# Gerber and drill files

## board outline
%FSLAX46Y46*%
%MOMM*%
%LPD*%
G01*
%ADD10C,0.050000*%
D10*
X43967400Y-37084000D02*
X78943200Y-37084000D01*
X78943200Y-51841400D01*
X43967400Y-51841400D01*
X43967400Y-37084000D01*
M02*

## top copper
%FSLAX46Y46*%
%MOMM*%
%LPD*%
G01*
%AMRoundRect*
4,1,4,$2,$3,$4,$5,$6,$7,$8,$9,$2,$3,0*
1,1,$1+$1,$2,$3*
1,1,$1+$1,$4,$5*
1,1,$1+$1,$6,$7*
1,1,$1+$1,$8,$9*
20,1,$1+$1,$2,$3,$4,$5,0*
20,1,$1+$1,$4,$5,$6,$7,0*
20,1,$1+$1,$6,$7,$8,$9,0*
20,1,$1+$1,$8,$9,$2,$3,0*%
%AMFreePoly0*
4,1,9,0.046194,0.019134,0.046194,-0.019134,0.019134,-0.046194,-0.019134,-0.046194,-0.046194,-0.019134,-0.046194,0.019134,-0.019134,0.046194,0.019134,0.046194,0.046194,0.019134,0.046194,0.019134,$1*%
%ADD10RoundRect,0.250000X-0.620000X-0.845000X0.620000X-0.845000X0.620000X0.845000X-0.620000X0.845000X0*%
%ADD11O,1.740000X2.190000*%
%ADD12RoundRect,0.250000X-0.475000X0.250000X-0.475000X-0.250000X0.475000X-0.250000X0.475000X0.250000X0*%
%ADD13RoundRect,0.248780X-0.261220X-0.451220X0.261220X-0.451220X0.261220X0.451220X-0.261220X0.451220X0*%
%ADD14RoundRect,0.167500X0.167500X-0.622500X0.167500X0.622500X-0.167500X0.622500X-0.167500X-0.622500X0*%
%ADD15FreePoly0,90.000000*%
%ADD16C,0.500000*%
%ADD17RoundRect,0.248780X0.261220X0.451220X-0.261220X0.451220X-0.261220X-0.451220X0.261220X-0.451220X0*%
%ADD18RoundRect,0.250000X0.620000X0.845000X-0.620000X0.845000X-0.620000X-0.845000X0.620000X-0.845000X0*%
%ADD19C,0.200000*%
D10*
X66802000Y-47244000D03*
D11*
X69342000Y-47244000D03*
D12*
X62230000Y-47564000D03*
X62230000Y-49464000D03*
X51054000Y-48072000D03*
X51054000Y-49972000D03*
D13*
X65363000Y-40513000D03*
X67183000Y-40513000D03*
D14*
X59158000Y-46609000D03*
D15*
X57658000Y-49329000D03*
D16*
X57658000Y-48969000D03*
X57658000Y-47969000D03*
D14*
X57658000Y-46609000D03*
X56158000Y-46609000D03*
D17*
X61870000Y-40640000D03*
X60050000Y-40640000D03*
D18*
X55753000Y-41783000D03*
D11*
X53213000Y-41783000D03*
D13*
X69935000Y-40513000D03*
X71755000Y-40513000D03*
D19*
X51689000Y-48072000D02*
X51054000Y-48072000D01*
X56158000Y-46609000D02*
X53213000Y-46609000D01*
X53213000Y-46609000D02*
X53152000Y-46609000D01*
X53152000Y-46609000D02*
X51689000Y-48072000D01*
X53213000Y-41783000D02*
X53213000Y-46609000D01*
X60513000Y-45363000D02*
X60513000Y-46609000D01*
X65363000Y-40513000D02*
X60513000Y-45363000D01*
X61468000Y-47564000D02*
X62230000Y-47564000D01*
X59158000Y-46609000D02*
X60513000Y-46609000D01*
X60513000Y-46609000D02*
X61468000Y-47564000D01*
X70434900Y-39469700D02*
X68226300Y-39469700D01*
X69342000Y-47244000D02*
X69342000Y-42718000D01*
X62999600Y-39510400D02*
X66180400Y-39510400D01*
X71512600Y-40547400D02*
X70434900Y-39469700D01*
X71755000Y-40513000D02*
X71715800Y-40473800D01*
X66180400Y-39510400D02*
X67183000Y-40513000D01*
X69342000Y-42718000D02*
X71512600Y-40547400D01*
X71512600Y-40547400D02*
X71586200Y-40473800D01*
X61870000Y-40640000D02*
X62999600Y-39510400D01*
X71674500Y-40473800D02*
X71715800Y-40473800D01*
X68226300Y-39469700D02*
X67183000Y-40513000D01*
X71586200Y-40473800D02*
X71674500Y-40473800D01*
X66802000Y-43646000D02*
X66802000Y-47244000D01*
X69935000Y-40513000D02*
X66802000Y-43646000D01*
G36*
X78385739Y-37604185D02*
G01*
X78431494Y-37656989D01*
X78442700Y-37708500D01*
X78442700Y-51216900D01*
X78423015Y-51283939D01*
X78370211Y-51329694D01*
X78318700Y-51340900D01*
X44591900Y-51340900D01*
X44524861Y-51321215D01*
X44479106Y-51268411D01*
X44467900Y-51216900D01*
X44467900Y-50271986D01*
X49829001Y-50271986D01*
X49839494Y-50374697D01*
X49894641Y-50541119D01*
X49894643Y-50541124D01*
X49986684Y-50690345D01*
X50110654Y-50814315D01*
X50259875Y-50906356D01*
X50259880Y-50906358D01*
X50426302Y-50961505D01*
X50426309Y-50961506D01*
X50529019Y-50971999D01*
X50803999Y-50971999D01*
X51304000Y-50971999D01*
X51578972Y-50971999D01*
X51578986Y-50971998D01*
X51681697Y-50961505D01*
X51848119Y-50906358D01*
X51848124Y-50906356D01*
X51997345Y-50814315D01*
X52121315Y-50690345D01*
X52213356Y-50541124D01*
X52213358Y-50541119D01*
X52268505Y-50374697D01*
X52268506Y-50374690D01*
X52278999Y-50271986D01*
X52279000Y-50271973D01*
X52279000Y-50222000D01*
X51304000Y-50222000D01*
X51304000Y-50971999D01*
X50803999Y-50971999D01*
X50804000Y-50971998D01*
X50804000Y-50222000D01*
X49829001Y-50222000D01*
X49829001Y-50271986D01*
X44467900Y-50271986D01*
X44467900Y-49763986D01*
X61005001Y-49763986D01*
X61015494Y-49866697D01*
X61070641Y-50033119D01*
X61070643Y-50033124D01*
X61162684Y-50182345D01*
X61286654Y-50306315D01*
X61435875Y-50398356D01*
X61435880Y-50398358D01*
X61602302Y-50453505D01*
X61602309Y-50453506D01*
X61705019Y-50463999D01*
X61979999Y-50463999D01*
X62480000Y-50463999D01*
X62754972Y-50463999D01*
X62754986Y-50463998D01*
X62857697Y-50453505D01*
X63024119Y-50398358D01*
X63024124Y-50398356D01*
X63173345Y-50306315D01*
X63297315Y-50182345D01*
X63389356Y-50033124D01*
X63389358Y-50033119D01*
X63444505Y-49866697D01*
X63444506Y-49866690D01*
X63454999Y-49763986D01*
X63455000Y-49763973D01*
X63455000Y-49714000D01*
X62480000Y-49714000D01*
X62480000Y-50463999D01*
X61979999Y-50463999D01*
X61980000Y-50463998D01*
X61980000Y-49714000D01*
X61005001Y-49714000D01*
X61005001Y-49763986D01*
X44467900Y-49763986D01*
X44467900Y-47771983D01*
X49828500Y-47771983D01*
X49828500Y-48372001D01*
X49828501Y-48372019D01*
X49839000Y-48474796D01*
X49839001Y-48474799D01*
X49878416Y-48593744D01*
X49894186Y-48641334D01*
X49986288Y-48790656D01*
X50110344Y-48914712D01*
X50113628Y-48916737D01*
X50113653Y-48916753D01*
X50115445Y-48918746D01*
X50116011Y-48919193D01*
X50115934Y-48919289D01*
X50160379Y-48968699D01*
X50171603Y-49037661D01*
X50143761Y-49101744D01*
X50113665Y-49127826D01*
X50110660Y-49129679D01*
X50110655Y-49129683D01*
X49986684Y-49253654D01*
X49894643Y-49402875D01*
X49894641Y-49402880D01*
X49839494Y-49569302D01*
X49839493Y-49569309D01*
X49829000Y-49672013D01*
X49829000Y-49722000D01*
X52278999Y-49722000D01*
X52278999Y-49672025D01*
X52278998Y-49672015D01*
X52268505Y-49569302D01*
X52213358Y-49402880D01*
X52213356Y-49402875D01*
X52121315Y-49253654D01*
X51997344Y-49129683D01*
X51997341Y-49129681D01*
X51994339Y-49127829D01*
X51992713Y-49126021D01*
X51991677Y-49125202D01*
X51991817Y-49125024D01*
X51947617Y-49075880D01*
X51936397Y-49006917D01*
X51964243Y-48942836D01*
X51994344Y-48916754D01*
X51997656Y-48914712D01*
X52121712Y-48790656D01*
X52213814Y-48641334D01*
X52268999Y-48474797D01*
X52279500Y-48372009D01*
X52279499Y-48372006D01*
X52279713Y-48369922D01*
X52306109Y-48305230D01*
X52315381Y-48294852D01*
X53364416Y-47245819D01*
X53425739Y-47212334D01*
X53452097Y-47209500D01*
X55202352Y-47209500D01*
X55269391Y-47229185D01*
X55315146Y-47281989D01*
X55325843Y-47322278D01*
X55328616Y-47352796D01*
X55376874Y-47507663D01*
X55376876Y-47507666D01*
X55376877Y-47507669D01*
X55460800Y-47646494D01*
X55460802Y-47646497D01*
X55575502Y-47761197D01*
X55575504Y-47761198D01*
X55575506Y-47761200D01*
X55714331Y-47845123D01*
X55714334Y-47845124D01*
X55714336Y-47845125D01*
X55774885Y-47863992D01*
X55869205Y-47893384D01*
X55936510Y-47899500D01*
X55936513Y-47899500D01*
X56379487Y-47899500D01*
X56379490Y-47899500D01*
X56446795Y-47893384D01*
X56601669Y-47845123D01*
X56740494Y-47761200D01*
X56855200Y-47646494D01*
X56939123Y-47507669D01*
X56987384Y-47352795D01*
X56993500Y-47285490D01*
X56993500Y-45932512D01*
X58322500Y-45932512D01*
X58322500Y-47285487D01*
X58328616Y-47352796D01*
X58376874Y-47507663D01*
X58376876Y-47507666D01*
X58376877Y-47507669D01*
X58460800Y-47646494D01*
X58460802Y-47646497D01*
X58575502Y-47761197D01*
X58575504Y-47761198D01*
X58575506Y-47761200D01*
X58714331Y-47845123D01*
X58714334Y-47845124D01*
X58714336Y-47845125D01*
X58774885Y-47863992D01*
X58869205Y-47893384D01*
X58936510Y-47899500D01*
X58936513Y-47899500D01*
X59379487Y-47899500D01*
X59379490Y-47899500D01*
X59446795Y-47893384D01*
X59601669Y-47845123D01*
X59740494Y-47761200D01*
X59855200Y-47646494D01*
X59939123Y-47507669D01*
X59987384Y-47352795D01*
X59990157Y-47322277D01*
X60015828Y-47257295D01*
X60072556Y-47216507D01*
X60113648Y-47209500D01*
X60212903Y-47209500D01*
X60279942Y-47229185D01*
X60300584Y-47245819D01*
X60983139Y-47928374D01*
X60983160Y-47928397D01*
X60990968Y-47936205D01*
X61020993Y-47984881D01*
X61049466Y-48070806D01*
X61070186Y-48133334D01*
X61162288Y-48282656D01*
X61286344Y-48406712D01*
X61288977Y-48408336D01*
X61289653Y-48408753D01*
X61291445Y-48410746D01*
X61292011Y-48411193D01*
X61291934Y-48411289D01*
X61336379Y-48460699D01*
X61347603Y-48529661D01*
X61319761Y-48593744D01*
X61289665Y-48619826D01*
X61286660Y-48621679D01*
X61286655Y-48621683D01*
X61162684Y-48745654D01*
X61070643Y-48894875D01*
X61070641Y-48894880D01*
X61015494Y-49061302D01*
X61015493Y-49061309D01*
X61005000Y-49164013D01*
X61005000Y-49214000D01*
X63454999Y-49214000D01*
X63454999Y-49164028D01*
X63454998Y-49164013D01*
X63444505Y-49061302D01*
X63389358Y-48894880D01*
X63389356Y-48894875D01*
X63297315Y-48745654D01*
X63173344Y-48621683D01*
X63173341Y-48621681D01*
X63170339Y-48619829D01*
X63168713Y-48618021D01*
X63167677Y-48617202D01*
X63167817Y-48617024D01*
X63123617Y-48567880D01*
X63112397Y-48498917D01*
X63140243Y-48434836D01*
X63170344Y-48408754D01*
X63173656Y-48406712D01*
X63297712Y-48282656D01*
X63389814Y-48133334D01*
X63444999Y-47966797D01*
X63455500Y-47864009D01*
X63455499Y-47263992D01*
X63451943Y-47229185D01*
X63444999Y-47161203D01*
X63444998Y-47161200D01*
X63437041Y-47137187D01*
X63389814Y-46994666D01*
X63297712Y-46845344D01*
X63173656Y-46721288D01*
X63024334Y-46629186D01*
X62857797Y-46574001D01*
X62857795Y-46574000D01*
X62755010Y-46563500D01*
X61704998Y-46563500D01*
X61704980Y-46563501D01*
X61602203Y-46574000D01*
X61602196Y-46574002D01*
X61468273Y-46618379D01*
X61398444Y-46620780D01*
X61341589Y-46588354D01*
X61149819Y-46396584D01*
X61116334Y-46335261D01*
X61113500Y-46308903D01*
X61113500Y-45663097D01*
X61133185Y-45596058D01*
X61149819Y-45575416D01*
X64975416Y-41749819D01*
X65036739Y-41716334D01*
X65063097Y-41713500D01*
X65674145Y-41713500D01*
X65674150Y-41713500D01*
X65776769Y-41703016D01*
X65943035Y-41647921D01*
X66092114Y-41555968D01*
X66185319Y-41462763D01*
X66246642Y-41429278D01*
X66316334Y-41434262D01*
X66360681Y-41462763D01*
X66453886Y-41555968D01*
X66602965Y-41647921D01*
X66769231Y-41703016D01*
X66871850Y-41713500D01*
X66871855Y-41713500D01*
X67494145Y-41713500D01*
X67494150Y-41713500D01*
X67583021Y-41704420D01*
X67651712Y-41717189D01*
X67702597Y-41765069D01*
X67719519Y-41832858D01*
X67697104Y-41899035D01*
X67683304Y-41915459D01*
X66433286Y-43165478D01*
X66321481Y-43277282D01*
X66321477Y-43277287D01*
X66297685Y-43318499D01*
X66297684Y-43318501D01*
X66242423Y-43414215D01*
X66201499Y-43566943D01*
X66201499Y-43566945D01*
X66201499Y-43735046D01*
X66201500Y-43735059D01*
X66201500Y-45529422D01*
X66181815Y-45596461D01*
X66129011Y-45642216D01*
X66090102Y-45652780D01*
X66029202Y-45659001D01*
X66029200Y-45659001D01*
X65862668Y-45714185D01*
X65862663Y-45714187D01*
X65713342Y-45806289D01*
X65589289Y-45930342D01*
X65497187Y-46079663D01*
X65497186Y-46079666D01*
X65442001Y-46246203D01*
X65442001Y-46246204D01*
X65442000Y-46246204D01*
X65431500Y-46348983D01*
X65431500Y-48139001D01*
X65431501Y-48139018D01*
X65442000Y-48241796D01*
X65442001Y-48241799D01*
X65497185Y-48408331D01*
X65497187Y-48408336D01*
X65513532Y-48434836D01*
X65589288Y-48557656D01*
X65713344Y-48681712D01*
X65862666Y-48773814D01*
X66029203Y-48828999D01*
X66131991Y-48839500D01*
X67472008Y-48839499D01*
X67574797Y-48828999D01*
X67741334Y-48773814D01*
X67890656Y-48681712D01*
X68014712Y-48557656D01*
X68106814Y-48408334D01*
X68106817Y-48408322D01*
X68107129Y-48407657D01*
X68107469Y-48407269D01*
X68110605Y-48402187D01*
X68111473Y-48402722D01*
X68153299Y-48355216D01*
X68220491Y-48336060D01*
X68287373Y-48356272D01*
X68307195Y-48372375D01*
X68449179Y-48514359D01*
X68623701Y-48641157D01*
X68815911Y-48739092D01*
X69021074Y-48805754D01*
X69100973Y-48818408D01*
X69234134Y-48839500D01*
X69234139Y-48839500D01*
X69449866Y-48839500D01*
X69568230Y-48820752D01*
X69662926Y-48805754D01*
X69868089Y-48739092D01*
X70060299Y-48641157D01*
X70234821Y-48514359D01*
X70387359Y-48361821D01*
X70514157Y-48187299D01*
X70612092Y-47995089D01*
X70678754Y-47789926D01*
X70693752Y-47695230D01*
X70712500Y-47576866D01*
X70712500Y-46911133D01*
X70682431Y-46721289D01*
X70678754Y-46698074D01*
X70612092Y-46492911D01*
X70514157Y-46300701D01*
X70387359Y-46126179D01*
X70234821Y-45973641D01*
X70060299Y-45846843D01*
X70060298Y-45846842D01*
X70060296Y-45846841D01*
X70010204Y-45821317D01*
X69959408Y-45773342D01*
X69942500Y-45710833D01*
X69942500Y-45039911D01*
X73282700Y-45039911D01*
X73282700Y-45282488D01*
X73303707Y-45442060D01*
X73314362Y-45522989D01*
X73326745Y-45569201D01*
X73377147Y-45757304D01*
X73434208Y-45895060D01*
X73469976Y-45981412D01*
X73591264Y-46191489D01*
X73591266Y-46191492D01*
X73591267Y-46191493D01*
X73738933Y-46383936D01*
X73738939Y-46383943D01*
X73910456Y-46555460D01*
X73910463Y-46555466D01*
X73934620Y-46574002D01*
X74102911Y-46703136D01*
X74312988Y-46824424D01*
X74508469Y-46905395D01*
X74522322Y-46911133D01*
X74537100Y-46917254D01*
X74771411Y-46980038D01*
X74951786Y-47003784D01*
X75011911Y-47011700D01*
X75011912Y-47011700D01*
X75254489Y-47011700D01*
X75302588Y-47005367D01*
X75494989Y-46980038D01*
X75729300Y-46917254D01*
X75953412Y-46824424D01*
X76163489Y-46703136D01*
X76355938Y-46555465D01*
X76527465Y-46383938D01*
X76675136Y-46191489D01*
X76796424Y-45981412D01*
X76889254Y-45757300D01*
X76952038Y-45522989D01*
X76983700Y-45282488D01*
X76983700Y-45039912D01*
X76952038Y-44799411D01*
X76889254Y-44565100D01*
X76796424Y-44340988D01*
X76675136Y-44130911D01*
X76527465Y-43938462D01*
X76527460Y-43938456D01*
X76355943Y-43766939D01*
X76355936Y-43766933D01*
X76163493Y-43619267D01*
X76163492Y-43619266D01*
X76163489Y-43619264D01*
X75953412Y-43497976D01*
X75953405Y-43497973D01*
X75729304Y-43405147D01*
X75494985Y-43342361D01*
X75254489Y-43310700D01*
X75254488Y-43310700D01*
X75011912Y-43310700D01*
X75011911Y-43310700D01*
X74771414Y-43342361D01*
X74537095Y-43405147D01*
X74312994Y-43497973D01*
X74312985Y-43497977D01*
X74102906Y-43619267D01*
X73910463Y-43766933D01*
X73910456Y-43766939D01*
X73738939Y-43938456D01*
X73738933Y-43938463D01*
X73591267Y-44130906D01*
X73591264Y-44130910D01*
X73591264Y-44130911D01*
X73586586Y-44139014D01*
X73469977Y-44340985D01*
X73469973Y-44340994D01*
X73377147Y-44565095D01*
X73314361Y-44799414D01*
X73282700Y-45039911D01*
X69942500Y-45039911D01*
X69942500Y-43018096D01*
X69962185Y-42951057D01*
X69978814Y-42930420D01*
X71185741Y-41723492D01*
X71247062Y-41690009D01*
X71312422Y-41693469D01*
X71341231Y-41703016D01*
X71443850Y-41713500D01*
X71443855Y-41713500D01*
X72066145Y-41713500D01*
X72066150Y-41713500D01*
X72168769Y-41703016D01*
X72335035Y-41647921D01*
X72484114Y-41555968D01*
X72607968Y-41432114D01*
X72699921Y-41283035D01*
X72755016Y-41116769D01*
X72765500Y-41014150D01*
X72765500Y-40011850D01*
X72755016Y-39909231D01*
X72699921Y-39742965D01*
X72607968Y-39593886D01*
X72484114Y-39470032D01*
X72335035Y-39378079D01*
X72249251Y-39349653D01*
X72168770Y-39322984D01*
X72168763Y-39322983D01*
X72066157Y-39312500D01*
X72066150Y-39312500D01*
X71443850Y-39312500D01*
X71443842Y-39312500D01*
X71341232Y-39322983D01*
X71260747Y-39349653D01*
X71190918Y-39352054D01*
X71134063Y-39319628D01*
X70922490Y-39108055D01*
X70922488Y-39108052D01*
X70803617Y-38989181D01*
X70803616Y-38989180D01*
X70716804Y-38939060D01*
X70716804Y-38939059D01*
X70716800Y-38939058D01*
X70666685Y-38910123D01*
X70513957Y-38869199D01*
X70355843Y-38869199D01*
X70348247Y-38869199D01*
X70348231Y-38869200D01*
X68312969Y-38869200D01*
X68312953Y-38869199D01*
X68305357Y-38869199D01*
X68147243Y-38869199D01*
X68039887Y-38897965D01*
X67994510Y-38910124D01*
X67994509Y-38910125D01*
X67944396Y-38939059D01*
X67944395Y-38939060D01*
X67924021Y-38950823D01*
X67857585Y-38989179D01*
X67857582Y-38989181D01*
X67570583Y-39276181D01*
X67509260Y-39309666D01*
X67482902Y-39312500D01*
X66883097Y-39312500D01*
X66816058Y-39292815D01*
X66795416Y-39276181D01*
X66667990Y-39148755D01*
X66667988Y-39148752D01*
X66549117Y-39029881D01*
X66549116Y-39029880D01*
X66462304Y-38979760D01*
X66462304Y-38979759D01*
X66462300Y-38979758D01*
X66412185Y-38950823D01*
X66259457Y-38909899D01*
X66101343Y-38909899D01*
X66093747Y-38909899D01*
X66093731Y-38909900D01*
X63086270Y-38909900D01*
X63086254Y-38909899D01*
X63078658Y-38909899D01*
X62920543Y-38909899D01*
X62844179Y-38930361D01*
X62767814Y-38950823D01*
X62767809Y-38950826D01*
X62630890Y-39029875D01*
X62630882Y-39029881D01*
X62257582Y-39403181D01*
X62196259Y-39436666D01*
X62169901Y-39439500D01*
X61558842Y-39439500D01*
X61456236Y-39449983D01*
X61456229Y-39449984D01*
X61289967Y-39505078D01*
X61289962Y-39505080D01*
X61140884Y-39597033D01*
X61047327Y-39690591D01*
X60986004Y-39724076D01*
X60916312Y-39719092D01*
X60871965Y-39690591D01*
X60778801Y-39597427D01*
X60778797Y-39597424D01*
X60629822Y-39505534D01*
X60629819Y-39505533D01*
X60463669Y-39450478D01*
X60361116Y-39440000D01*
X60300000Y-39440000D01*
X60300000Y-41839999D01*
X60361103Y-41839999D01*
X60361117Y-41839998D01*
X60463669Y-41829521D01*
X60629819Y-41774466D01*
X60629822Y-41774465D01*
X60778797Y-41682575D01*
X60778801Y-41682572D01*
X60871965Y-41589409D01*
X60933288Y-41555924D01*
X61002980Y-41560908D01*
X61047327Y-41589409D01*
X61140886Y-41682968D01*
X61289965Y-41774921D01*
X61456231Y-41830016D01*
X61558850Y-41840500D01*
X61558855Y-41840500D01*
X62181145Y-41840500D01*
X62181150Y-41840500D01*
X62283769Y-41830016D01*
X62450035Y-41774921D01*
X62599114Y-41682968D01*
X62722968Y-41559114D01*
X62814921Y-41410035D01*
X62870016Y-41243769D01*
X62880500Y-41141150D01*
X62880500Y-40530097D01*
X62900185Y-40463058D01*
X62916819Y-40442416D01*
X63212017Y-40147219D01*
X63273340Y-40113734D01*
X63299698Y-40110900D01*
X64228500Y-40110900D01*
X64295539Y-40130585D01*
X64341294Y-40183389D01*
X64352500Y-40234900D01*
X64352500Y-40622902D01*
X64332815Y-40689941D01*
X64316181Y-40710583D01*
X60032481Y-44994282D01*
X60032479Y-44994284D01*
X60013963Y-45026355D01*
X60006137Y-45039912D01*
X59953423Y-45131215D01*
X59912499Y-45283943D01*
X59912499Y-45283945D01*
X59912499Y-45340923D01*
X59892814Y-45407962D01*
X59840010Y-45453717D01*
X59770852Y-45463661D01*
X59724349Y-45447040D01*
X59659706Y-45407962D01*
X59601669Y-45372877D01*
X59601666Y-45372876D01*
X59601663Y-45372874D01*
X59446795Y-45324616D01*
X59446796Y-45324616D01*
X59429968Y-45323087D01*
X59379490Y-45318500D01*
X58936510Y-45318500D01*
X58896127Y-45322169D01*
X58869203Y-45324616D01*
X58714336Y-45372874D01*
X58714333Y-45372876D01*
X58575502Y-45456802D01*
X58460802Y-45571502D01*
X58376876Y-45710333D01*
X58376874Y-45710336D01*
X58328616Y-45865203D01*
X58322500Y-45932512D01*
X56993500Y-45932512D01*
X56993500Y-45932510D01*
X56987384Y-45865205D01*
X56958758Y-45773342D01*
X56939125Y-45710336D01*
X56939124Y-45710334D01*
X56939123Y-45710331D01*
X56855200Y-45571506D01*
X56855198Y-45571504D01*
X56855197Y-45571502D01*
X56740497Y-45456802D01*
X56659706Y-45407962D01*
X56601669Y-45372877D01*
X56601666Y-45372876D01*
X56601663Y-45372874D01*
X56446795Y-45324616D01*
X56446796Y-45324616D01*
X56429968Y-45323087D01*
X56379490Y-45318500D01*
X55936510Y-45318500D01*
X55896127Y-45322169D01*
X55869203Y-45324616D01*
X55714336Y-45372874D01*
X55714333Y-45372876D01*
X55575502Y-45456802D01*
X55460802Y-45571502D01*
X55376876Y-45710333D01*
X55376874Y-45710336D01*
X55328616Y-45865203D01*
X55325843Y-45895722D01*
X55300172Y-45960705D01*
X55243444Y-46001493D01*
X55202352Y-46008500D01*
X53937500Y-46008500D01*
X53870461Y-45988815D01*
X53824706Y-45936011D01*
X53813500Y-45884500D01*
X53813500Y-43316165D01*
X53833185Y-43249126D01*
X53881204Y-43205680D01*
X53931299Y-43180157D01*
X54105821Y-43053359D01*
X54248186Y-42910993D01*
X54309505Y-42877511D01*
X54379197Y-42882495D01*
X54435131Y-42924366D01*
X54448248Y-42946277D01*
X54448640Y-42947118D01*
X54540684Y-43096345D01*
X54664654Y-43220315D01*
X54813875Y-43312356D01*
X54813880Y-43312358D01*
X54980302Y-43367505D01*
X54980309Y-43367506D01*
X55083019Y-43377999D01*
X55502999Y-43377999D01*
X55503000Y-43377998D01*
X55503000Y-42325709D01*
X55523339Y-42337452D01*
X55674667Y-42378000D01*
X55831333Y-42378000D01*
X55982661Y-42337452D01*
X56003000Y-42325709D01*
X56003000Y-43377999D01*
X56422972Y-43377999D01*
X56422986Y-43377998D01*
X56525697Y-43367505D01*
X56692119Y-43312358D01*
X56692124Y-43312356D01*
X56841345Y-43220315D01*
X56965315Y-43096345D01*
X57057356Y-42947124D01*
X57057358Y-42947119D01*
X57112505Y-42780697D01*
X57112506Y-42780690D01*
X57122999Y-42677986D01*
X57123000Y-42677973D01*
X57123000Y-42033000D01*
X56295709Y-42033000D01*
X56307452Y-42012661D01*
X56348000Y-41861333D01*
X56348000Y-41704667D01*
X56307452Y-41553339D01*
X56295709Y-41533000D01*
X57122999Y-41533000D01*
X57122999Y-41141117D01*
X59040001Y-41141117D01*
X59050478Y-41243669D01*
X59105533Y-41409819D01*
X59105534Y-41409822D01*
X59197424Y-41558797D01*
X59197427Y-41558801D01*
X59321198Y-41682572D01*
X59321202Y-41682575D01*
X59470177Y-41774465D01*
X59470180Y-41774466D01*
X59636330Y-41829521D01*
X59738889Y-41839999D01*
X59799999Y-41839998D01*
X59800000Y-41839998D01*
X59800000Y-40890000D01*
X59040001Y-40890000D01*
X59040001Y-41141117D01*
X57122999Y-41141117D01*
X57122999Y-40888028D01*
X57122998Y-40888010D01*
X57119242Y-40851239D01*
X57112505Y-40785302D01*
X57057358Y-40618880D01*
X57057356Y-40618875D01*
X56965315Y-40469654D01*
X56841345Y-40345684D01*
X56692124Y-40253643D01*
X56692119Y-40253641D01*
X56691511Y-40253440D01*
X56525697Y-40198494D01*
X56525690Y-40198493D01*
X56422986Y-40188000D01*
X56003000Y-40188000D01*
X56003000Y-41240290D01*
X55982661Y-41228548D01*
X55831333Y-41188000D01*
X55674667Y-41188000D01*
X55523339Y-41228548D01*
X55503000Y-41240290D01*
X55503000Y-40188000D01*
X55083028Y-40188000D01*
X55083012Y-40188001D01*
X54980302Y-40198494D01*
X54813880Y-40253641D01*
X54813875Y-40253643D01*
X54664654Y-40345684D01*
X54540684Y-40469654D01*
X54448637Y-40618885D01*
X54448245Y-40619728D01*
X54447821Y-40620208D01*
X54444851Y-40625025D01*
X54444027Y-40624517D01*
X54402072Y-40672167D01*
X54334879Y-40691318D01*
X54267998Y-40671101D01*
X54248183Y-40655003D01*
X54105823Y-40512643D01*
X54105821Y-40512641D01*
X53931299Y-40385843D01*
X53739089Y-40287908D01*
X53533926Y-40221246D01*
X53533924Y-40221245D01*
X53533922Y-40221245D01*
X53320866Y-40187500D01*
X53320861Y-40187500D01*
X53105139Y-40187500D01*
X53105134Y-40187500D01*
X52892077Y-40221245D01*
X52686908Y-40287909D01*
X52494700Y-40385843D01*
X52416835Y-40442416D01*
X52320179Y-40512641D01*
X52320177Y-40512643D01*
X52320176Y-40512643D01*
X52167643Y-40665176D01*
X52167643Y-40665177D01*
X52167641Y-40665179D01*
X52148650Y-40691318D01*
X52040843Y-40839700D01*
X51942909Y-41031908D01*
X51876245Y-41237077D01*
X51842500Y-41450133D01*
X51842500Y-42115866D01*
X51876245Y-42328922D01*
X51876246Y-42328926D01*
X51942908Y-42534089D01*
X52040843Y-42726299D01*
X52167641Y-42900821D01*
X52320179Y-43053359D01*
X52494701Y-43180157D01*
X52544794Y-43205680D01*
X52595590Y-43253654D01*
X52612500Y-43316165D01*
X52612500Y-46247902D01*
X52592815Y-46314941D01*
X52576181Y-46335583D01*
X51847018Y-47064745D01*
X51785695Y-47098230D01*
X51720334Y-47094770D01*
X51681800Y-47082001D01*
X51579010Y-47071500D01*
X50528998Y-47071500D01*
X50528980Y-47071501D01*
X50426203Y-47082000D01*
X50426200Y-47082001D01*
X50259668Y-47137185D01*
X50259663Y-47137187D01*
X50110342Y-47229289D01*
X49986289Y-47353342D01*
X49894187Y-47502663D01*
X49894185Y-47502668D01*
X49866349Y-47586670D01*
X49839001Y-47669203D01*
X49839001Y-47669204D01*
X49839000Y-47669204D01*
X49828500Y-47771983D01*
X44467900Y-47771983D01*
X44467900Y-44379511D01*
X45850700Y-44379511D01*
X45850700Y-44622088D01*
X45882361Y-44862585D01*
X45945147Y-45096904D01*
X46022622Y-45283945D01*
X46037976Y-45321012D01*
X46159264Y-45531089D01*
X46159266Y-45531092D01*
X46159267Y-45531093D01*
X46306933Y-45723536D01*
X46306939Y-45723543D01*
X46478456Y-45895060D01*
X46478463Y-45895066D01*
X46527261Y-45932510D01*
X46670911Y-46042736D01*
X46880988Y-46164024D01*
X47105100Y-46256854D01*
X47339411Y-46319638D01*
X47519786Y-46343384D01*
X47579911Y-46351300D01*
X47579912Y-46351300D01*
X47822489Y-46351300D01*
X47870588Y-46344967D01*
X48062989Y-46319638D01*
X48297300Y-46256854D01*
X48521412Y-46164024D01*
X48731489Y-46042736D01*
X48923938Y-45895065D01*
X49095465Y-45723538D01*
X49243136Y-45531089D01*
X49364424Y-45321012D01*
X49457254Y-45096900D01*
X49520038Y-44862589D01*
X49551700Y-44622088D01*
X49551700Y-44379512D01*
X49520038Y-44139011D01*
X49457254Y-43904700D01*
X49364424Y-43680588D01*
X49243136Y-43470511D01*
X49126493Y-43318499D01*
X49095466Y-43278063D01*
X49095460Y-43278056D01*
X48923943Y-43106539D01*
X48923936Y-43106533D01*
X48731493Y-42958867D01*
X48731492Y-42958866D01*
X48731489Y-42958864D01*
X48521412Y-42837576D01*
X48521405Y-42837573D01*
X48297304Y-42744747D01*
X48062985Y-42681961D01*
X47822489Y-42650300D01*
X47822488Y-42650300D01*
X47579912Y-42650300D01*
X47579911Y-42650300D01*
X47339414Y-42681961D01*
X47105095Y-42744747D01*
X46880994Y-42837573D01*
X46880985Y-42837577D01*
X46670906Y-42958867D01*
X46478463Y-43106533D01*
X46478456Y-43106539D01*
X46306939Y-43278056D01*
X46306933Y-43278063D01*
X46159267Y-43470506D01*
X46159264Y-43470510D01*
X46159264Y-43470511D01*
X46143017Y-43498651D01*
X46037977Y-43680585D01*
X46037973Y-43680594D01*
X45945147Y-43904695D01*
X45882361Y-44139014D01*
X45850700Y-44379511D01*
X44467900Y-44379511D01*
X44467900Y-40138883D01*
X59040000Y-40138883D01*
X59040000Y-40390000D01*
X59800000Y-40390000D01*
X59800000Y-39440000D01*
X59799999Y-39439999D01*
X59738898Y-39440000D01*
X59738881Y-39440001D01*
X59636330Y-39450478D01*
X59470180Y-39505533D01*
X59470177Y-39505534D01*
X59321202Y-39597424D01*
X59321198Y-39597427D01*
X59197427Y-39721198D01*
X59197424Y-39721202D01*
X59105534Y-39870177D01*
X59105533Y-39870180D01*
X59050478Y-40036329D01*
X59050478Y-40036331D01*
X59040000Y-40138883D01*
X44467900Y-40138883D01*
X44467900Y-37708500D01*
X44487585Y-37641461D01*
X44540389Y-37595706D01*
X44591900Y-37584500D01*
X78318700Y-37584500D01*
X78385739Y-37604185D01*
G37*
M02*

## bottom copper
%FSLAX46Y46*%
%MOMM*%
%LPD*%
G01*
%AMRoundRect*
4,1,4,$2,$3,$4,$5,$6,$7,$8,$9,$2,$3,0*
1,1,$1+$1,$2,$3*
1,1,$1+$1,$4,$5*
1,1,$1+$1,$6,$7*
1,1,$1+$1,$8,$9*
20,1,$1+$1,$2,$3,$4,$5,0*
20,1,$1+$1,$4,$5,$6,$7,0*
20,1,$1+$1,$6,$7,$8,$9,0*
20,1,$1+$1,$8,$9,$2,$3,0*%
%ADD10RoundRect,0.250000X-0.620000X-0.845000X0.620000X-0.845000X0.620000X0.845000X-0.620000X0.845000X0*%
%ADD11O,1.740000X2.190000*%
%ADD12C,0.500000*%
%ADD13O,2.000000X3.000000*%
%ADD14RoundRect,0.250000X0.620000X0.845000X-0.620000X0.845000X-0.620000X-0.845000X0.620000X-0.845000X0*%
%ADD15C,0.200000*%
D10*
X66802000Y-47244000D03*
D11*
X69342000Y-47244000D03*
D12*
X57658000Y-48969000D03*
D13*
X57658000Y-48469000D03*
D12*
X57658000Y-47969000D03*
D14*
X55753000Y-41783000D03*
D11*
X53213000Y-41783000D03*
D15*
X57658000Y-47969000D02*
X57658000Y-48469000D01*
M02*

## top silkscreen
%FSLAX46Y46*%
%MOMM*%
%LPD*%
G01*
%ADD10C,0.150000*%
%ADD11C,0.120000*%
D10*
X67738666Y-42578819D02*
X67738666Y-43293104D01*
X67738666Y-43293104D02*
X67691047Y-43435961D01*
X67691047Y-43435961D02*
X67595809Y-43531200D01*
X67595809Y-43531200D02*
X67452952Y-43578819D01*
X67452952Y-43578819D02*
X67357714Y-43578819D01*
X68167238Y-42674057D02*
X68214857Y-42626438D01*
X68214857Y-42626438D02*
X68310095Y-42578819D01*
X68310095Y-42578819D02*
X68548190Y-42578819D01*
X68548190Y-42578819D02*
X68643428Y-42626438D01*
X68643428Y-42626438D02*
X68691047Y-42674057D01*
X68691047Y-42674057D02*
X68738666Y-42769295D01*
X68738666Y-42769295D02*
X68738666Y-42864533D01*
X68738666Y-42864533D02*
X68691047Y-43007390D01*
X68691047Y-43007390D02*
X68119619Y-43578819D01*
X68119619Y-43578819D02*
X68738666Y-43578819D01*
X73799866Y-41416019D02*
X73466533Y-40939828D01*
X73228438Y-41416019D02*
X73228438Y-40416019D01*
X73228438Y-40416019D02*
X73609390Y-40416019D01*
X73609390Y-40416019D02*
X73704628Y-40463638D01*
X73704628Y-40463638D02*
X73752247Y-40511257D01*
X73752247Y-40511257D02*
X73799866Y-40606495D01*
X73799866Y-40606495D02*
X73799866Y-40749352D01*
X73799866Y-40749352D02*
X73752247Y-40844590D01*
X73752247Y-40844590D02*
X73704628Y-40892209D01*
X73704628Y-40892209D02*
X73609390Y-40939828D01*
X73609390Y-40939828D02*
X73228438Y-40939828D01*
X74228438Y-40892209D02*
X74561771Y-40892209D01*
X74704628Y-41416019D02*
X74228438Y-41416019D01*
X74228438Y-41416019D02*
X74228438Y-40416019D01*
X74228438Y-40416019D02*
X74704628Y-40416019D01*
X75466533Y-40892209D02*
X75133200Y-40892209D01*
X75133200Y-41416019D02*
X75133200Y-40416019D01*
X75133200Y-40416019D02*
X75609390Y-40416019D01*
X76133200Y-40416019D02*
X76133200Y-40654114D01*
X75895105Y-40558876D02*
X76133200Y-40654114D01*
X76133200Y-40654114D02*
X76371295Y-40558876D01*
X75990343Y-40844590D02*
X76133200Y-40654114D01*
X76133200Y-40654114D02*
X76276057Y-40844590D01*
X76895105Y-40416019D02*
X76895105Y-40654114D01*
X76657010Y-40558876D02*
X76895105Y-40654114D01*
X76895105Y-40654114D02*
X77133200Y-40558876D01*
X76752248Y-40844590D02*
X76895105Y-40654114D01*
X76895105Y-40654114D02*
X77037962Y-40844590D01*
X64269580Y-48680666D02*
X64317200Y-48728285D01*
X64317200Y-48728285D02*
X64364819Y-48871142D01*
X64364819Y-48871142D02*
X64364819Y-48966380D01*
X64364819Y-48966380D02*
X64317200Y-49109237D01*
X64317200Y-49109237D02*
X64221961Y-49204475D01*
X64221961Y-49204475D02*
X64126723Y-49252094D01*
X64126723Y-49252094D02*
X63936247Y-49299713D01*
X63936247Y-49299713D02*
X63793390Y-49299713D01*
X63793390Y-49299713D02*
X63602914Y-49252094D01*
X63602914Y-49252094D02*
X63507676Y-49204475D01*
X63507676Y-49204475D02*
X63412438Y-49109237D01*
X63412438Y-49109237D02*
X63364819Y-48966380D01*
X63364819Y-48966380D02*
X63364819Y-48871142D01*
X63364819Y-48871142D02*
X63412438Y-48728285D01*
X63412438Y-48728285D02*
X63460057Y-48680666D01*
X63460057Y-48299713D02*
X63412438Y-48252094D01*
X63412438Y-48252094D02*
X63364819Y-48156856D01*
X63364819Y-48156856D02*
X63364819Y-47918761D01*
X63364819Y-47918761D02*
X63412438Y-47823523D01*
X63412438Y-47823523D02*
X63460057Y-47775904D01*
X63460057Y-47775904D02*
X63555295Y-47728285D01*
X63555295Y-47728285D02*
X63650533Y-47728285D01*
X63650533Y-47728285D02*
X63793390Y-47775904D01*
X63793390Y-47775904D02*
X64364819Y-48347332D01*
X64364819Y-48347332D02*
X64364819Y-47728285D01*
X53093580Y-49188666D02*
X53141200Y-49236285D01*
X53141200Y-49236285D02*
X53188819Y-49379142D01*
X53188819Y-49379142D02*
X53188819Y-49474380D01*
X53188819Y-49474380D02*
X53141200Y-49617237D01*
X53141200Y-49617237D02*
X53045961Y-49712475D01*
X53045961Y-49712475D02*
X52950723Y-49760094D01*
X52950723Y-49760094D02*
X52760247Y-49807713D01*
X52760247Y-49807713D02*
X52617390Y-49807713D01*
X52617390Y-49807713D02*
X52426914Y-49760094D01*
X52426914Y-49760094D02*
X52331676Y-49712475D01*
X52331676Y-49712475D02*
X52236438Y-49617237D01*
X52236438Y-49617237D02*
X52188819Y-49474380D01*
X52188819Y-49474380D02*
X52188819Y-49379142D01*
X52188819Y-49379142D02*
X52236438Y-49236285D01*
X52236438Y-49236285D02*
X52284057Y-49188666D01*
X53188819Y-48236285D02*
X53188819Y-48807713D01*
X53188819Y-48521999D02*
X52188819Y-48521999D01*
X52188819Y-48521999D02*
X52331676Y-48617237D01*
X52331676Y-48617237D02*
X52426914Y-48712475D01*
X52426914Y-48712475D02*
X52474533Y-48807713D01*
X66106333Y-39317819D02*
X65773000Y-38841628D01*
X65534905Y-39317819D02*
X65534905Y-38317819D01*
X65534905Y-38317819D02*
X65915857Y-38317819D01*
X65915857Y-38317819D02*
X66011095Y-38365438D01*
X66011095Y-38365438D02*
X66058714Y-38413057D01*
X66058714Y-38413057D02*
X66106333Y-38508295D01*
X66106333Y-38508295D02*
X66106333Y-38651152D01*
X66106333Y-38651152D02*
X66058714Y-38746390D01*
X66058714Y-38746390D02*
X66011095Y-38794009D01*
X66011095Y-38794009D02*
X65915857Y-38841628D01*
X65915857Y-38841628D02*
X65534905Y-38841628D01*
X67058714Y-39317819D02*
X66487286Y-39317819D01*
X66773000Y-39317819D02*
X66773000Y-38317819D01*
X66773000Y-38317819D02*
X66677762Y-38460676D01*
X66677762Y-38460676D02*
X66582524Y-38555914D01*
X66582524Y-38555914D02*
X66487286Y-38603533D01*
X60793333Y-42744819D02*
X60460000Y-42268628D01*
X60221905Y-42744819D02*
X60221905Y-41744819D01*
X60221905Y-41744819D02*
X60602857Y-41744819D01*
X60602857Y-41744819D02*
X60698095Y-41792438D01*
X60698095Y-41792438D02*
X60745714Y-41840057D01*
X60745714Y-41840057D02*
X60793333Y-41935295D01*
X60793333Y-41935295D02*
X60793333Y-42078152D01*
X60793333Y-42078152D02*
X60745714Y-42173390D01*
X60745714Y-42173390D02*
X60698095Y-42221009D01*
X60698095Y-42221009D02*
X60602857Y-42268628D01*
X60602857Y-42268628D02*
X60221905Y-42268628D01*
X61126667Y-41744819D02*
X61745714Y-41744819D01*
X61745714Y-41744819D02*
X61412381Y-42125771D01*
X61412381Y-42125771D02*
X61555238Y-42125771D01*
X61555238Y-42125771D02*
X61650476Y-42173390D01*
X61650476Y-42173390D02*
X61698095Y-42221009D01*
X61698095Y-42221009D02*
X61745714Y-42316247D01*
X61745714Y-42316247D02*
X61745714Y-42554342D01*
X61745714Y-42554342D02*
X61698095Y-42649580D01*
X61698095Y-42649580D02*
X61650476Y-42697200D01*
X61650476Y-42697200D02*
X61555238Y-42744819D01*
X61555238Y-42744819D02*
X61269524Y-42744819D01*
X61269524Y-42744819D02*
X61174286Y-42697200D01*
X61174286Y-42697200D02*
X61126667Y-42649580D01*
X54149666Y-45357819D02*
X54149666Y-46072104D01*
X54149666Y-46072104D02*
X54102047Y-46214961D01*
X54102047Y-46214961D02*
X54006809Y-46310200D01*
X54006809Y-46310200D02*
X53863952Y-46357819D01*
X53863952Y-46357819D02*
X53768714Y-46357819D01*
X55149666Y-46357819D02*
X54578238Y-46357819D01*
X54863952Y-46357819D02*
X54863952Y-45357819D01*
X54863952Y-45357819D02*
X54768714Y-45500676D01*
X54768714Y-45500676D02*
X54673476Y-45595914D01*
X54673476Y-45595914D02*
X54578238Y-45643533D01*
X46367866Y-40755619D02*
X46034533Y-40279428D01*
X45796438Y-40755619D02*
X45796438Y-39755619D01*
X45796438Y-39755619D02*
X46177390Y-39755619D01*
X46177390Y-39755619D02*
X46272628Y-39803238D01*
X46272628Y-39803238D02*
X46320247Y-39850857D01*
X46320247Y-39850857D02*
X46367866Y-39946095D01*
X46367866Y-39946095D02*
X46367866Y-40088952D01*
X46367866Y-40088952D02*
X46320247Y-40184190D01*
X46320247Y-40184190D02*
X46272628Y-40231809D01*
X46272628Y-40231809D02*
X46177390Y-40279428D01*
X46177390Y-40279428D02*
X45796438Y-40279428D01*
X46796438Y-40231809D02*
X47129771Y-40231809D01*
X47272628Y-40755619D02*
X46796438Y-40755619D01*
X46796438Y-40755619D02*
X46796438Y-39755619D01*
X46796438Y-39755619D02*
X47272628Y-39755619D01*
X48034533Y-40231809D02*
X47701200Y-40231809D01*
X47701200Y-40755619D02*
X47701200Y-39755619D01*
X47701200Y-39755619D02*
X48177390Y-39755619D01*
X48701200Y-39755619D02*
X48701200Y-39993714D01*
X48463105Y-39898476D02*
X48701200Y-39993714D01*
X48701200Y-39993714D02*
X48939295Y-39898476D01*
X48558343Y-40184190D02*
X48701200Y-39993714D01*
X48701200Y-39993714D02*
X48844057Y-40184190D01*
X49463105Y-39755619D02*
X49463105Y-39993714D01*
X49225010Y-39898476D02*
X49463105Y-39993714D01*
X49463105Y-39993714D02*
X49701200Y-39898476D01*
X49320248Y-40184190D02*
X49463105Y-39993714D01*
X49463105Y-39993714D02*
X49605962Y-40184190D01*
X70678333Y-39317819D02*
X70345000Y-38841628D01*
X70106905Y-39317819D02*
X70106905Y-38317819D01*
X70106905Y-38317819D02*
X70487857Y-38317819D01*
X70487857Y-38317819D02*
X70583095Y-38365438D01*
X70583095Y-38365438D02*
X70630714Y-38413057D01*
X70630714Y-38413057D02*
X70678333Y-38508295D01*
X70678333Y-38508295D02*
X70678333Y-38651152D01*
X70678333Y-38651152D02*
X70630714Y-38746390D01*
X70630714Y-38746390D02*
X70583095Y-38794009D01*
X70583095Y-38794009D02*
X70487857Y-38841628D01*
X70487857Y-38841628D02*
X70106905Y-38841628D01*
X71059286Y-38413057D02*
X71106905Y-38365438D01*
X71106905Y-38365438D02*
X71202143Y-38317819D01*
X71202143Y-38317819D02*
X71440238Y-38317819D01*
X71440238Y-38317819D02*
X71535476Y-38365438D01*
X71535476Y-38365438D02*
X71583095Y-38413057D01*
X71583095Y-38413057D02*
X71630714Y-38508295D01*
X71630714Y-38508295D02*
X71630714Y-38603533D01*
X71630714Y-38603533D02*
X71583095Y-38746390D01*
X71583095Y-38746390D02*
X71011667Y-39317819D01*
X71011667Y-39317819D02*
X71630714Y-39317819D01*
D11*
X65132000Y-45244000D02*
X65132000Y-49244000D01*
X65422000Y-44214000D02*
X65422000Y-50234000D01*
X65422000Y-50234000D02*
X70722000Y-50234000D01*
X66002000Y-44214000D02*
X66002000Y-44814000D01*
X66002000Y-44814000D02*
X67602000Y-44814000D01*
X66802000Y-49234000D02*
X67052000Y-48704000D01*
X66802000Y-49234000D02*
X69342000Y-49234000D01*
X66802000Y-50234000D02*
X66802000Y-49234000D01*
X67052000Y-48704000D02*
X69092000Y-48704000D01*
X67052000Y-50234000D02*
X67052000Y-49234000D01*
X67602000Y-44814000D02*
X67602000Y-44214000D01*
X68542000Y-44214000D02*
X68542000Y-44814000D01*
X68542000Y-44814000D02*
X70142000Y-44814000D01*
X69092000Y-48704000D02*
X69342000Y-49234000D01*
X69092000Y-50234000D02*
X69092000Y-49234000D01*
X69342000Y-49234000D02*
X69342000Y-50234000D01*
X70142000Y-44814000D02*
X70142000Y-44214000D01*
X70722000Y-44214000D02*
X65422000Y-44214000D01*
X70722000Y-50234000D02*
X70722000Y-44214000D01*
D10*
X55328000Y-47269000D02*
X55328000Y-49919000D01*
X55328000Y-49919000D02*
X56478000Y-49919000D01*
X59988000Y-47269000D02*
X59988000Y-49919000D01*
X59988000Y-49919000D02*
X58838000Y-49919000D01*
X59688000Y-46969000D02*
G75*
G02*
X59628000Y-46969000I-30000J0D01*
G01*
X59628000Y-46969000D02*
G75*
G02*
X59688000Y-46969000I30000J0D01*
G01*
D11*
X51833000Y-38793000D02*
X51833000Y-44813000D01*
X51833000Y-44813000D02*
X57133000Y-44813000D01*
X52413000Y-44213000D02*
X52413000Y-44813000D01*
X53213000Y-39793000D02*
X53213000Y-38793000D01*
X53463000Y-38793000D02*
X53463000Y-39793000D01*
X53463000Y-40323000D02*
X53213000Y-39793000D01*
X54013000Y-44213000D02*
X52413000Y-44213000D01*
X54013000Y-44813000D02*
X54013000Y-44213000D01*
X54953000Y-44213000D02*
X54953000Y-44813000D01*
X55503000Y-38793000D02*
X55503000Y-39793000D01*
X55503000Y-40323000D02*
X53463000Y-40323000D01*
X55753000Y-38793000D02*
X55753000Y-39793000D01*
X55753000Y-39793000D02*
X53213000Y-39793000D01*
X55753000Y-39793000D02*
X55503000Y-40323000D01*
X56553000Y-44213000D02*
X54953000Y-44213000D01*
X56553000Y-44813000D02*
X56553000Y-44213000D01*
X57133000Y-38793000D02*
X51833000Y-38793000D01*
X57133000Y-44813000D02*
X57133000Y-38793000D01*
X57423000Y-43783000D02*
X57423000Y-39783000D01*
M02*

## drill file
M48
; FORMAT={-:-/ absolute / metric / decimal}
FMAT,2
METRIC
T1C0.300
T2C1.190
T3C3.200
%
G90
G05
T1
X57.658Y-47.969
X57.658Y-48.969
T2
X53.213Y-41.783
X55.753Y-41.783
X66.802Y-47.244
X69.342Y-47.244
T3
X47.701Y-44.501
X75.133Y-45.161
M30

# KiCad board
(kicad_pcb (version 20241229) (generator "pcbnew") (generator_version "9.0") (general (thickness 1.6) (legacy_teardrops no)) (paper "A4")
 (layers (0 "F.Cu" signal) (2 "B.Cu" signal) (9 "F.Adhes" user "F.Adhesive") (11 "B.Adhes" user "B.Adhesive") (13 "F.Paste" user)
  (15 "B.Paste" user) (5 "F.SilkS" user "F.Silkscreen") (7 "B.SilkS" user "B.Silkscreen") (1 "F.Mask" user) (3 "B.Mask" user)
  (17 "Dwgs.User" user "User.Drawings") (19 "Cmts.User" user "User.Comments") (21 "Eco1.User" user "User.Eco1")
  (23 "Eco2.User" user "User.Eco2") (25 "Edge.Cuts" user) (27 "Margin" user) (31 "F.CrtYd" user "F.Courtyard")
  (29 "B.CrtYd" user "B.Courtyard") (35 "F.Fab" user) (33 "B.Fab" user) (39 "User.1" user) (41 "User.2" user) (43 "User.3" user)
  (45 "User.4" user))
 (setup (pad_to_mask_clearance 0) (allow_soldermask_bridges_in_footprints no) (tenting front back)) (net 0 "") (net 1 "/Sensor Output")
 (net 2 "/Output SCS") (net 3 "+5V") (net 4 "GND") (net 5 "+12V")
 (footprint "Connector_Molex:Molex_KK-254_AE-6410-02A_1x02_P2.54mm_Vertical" (layer "F.Cu") (at 66.802 47.244)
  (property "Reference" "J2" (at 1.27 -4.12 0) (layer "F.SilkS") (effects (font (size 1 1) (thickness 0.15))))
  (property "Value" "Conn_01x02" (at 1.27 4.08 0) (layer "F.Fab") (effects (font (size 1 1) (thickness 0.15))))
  (fp_line (start -1.67 -2) (end -1.67 2) (stroke (width 0.12) (type solid)) (layer "F.SilkS"))
  (fp_line (start -1.38 -3.03) (end -1.38 2.99) (stroke (width 0.12) (type solid)) (layer "F.SilkS"))
  (fp_line (start -1.38 2.99) (end 3.92 2.99) (stroke (width 0.12) (type solid)) (layer "F.SilkS"))
  (fp_line (start -0.8 -3.03) (end -0.8 -2.43) (stroke (width 0.12) (type solid)) (layer "F.SilkS"))
  (fp_line (start -0.8 -2.43) (end 0.8 -2.43) (stroke (width 0.12) (type solid)) (layer "F.SilkS"))
  (fp_line (start 0 1.99) (end 0.25 1.46) (stroke (width 0.12) (type solid)) (layer "F.SilkS"))
  (fp_line (start 0 1.99) (end 2.54 1.99) (stroke (width 0.12) (type solid)) (layer "F.SilkS"))
  (fp_line (start 0 2.99) (end 0 1.99) (stroke (width 0.12) (type solid)) (layer "F.SilkS"))
  (fp_line (start 0.25 1.46) (end 2.29 1.46) (stroke (width 0.12) (type solid)) (layer "F.SilkS"))
  (fp_line (start 0.25 2.99) (end 0.25 1.99) (stroke (width 0.12) (type solid)) (layer "F.SilkS"))
  (fp_line (start 0.8 -2.43) (end 0.8 -3.03) (stroke (width 0.12) (type solid)) (layer "F.SilkS"))
  (fp_line (start 1.74 -3.03) (end 1.74 -2.43) (stroke (width 0.12) (type solid)) (layer "F.SilkS"))
  (fp_line (start 1.74 -2.43) (end 3.34 -2.43) (stroke (width 0.12) (type solid)) (layer "F.SilkS"))
  (fp_line (start 2.29 1.46) (end 2.54 1.99) (stroke (width 0.12) (type solid)) (layer "F.SilkS"))
  (fp_line (start 2.29 2.99) (end 2.29 1.99) (stroke (width 0.12) (type solid)) (layer "F.SilkS"))
  (fp_line (start 2.54 1.99) (end 2.54 2.99) (stroke (width 0.12) (type solid)) (layer "F.SilkS"))
  (fp_line (start 3.34 -2.43) (end 3.34 -3.03) (stroke (width 0.12) (type solid)) (layer "F.SilkS"))
  (fp_line (start 3.92 -3.03) (end -1.38 -3.03) (stroke (width 0.12) (type solid)) (layer "F.SilkS"))
  (fp_line (start 3.92 2.99) (end 3.92 -3.03) (stroke (width 0.12) (type solid)) (layer "F.SilkS"))
  (pad "1" thru_hole roundrect (at 0 0) (size 1.74 2.19) (drill 1.19) (layers "*.Cu" "*.Mask") (remove_unused_layers no)
   (roundrect_rratio 0.143678) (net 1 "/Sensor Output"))
  (pad "2" thru_hole oval (at 2.54 0) (size 1.74 2.19) (drill 1.19) (layers "*.Cu" "*.Mask") (remove_unused_layers no) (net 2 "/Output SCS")))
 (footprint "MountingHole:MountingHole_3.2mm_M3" (layer "F.Cu") (at 75.1332 45.1612)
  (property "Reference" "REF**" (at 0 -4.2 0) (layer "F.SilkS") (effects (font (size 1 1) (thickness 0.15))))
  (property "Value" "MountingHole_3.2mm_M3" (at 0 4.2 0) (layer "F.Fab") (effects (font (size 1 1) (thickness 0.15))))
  (pad "" np_thru_hole circle (at 0 0) (size 3.2 3.2) (drill 3.2) (layers "*.Cu" "*.Mask")))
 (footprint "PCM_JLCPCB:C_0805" (layer "F.Cu") (at 62.23 48.514 -90)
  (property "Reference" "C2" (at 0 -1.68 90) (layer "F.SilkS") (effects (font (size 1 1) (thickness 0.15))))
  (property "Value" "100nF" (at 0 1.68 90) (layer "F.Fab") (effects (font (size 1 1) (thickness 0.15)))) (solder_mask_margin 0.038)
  (pad "1" smd roundrect (at -0.95 0 270) (size 1 1.45) (layers "F.Cu" "F.Mask" "F.Paste") (roundrect_rratio 0.25) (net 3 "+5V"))
  (pad "2" smd roundrect (at 0.95 0 270) (size 1 1.45) (layers "F.Cu" "F.Mask" "F.Paste") (roundrect_rratio 0.25) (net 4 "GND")))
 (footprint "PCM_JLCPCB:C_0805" (layer "F.Cu") (at 51.054 49.022 -90)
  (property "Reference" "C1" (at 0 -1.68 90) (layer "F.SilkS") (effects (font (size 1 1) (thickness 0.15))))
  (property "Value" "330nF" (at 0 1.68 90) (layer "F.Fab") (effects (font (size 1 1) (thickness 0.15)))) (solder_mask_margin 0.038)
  (pad "1" smd roundrect (at -0.95 0 270) (size 1 1.45) (layers "F.Cu" "F.Mask" "F.Paste") (roundrect_rratio 0.25) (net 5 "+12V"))
  (pad "2" smd roundrect (at 0.95 0 270) (size 1 1.45) (layers "F.Cu" "F.Mask" "F.Paste") (roundrect_rratio 0.25) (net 4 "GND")))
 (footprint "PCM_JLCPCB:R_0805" (layer "F.Cu") (at 66.273 40.513)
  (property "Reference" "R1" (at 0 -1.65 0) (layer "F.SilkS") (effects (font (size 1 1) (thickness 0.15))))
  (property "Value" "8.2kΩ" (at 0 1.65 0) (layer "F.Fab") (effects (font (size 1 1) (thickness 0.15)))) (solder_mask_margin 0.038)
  (pad "1" smd roundrect (at -0.91 0) (size 1.02 1.4) (layers "F.Cu" "F.Mask" "F.Paste") (roundrect_rratio 0.243902) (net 3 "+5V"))
  (pad "2" smd roundrect (at 0.91 0) (size 1.02 1.4) (layers "F.Cu" "F.Mask" "F.Paste") (roundrect_rratio 0.243902) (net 2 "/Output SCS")))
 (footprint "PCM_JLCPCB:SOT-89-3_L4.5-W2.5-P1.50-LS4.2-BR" (layer "F.Cu") (at 57.658 47.969 90)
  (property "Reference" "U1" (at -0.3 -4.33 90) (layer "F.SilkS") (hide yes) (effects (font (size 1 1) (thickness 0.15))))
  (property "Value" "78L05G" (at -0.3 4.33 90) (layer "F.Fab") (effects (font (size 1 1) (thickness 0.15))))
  (fp_line (start 0.7 -2.33) (end -1.95 -2.33) (stroke (width 0.15) (type solid)) (layer "F.SilkS"))
  (fp_line (start -1.95 -2.33) (end -1.95 -1.18) (stroke (width 0.15) (type solid)) (layer "F.SilkS"))
  (fp_line (start 0.7 2.33) (end -1.95 2.33) (stroke (width 0.15) (type solid)) (layer "F.SilkS"))
  (fp_line (start -1.95 2.33) (end -1.95 1.18) (stroke (width 0.15) (type solid)) (layer "F.SilkS"))
  (fp_circle (center 1 2) (end 1.03 2) (stroke (width 0.15) (type solid)) (fill no) (layer "F.SilkS"))
  (pad "1" smd roundrect (at 1.36 1.5 90) (size 1.58 0.67) (layers "F.Cu" "F.Mask" "F.Paste") (roundrect_rratio 0.25) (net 3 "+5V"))
  (pad "2" smd custom (at -1.36 0 90) (size 0.1 0.1) (layers "F.Cu" "F.Mask" "F.Paste") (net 4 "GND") (zone_connect 2)
   (thermal_bridge_angle 90) (options (clearance outline) (anchor circle)) (primitives))
  (pad "2" thru_hole circle (at -1 0 90) (size 0.5 0.5) (drill 0.3) (layers "*.Cu" "F.Mask") (remove_unused_layers no) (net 4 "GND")
   (zone_connect 2))
  (pad "2" smd oval (at -0.5 0 90) (size 3 2) (layers "B.Cu") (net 4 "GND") (zone_connect 2) (thermal_bridge_angle 45))
  (pad "2" thru_hole circle (at 0 0 90) (size 0.5 0.5) (drill 0.3) (layers "*.Cu" "F.Mask") (remove_unused_layers no) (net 4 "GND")
   (zone_connect 2))
  (pad "2" smd roundrect (at 1.36 0 90) (size 1.58 0.67) (layers "F.Cu" "F.Mask" "F.Paste") (roundrect_rratio 0.25) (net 4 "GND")
   (zone_connect 2))
  (pad "3" smd roundrect (at 1.36 -1.5 90) (size 1.58 0.67) (layers "F.Cu" "F.Mask" "F.Paste") (roundrect_rratio 0.25) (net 5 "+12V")))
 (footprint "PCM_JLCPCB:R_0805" (layer "F.Cu") (at 60.96 40.64 180)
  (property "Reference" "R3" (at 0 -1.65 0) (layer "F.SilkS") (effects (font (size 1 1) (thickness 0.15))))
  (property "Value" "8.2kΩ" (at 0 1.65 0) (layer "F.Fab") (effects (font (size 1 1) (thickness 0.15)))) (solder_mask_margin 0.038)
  (pad "1" smd roundrect (at -0.91 0 180) (size 1.02 1.4) (layers "F.Cu" "F.Mask" "F.Paste") (roundrect_rratio 0.243902)
   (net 2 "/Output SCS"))
  (pad "2" smd roundrect (at 0.91 0 180) (size 1.02 1.4) (layers "F.Cu" "F.Mask" "F.Paste") (roundrect_rratio 0.243902) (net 4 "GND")))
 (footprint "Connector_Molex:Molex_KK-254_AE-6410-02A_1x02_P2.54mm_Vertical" (layer "F.Cu") (at 55.753 41.783 180)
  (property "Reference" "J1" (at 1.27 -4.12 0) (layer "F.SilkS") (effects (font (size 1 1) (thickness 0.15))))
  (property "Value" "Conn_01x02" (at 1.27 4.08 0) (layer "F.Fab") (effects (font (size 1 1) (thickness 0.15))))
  (fp_line (start 3.92 2.99) (end 3.92 -3.03) (stroke (width 0.12) (type solid)) (layer "F.SilkS"))
  (fp_line (start 3.92 -3.03) (end -1.38 -3.03) (stroke (width 0.12) (type solid)) (layer "F.SilkS"))
  (fp_line (start 3.34 -2.43) (end 3.34 -3.03) (stroke (width 0.12) (type solid)) (layer "F.SilkS"))
  (fp_line (start 2.54 1.99) (end 2.54 2.99) (stroke (width 0.12) (type solid)) (layer "F.SilkS"))
  (fp_line (start 2.29 2.99) (end 2.29 1.99) (stroke (width 0.12) (type solid)) (layer "F.SilkS"))
  (fp_line (start 2.29 1.46) (end 2.54 1.99) (stroke (width 0.12) (type solid)) (layer "F.SilkS"))
  (fp_line (start 1.74 -2.43) (end 3.34 -2.43) (stroke (width 0.12) (type solid)) (layer "F.SilkS"))
  (fp_line (start 1.74 -3.03) (end 1.74 -2.43) (stroke (width 0.12) (type solid)) (layer "F.SilkS"))
  (fp_line (start 0.8 -2.43) (end 0.8 -3.03) (stroke (width 0.12) (type solid)) (layer "F.SilkS"))
  (fp_line (start 0.25 2.99) (end 0.25 1.99) (stroke (width 0.12) (type solid)) (layer "F.SilkS"))
  (fp_line (start 0.25 1.46) (end 2.29 1.46) (stroke (width 0.12) (type solid)) (layer "F.SilkS"))
  (fp_line (start 0 2.99) (end 0 1.99) (stroke (width 0.12) (type solid)) (layer "F.SilkS"))
  (fp_line (start 0 1.99) (end 2.54 1.99) (stroke (width 0.12) (type solid)) (layer "F.SilkS"))
  (fp_line (start 0 1.99) (end 0.25 1.46) (stroke (width 0.12) (type solid)) (layer "F.SilkS"))
  (fp_line (start -0.8 -2.43) (end 0.8 -2.43) (stroke (width 0.12) (type solid)) (layer "F.SilkS"))
  (fp_line (start -0.8 -3.03) (end -0.8 -2.43) (stroke (width 0.12) (type solid)) (layer "F.SilkS"))
  (fp_line (start -1.38 2.99) (end 3.92 2.99) (stroke (width 0.12) (type solid)) (layer "F.SilkS"))
  (fp_line (start -1.38 -3.03) (end -1.38 2.99) (stroke (width 0.12) (type solid)) (layer "F.SilkS"))
  (fp_line (start -1.67 -2) (end -1.67 2) (stroke (width 0.12) (type solid)) (layer "F.SilkS"))
  (pad "1" thru_hole roundrect (at 0 0 180) (size 1.74 2.19) (drill 1.19) (layers "*.Cu" "*.Mask") (remove_unused_layers no)
   (roundrect_rratio 0.143678) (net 4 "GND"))
  (pad "2" thru_hole oval (at 2.54 0 180) (size 1.74 2.19) (drill 1.19) (layers "*.Cu" "*.Mask") (remove_unused_layers no) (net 5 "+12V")))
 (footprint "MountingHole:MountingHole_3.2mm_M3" (layer "F.Cu") (at 47.7012 44.5008)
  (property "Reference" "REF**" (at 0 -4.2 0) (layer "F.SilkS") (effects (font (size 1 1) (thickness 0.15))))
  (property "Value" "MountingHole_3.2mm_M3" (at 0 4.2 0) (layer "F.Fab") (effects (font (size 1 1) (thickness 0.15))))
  (pad "" np_thru_hole circle (at 0 0) (size 3.2 3.2) (drill 3.2) (layers "*.Cu" "*.Mask")))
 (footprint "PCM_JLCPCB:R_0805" (layer "F.Cu") (at 70.845 40.513)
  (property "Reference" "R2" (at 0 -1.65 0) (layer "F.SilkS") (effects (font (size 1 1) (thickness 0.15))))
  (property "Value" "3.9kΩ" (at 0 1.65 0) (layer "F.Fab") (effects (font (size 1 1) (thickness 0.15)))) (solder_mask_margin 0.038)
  (pad "1" smd roundrect (at -0.91 0) (size 1.02 1.4) (layers "F.Cu" "F.Mask" "F.Paste") (roundrect_rratio 0.243902)
   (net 1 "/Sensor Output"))
  (pad "2" smd roundrect (at 0.91 0) (size 1.02 1.4) (layers "F.Cu" "F.Mask" "F.Paste") (roundrect_rratio 0.243902) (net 2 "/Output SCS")))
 (gr_rect (start 43.9674 37.084) (end 78.9432 51.8414) (stroke (width 0.05) (type default)) (fill no) (layer "Edge.Cuts"))
 (segment (start 57.658 47.969) (end 57.658 48.469) (width 0.2) (layer "B.Cu") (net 4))
 (segment (start 51.689 48.072) (end 51.054 48.072) (width 0.2) (layer "F.Cu") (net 5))
 (segment (start 56.158 46.609) (end 53.213 46.609) (width 0.2) (layer "F.Cu") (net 5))
 (segment (start 53.213 46.609) (end 53.152 46.609) (width 0.2) (layer "F.Cu") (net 5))
 (segment (start 53.152 46.609) (end 51.689 48.072) (width 0.2) (layer "F.Cu") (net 5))
 (segment (start 53.213 41.783) (end 53.213 46.609) (width 0.2) (layer "F.Cu") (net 5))
 (segment (start 60.513 45.363) (end 60.513 46.609) (width 0.2) (layer "F.Cu") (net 3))
 (segment (start 65.363 40.513) (end 60.513 45.363) (width 0.2) (layer "F.Cu") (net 3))
 (segment (start 61.468 47.564) (end 62.23 47.564) (width 0.2) (layer "F.Cu") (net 3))
 (segment (start 59.158 46.609) (end 60.513 46.609) (width 0.2) (layer "F.Cu") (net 3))
 (segment (start 60.513 46.609) (end 61.468 47.564) (width 0.2) (layer "F.Cu") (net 3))
 (segment (start 70.4349 39.4697) (end 68.2263 39.4697) (width 0.2) (layer "F.Cu") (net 2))
 (segment (start 69.342 47.244) (end 69.342 42.718) (width 0.2) (layer "F.Cu") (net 2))
 (segment (start 62.9996 39.5104) (end 66.1804 39.5104) (width 0.2) (layer "F.Cu") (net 2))
 (segment (start 71.5126 40.5474) (end 70.4349 39.4697) (width 0.2) (layer "F.Cu") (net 2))
 (segment (start 71.755 40.513) (end 71.7158 40.4738) (width 0.2) (layer "F.Cu") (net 2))
 (segment (start 66.1804 39.5104) (end 67.183 40.513) (width 0.2) (layer "F.Cu") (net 2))
 (segment (start 69.342 42.718) (end 71.5126 40.5474) (width 0.2) (layer "F.Cu") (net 2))
 (segment (start 71.5126 40.5474) (end 71.5862 40.4738) (width 0.2) (layer "F.Cu") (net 2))
 (segment (start 61.87 40.64) (end 62.9996 39.5104) (width 0.2) (layer "F.Cu") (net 2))
 (segment (start 71.6745 40.4738) (end 71.7158 40.4738) (width 0.2) (layer "F.Cu") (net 2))
 (segment (start 68.2263 39.4697) (end 67.183 40.513) (width 0.2) (layer "F.Cu") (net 2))
 (segment (start 71.5862 40.4738) (end 71.6745 40.4738) (width 0.2) (layer "F.Cu") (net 2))
 (segment (start 66.802 43.646) (end 66.802 47.244) (width 0.2) (layer "F.Cu") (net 1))
 (segment (start 69.935 40.513) (end 66.802 43.646) (width 0.2) (layer "F.Cu") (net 1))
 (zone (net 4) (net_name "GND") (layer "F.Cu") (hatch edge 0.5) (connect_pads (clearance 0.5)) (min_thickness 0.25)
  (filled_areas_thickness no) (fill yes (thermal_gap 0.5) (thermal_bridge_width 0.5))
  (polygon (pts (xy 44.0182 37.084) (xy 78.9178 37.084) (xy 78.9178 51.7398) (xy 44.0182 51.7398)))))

